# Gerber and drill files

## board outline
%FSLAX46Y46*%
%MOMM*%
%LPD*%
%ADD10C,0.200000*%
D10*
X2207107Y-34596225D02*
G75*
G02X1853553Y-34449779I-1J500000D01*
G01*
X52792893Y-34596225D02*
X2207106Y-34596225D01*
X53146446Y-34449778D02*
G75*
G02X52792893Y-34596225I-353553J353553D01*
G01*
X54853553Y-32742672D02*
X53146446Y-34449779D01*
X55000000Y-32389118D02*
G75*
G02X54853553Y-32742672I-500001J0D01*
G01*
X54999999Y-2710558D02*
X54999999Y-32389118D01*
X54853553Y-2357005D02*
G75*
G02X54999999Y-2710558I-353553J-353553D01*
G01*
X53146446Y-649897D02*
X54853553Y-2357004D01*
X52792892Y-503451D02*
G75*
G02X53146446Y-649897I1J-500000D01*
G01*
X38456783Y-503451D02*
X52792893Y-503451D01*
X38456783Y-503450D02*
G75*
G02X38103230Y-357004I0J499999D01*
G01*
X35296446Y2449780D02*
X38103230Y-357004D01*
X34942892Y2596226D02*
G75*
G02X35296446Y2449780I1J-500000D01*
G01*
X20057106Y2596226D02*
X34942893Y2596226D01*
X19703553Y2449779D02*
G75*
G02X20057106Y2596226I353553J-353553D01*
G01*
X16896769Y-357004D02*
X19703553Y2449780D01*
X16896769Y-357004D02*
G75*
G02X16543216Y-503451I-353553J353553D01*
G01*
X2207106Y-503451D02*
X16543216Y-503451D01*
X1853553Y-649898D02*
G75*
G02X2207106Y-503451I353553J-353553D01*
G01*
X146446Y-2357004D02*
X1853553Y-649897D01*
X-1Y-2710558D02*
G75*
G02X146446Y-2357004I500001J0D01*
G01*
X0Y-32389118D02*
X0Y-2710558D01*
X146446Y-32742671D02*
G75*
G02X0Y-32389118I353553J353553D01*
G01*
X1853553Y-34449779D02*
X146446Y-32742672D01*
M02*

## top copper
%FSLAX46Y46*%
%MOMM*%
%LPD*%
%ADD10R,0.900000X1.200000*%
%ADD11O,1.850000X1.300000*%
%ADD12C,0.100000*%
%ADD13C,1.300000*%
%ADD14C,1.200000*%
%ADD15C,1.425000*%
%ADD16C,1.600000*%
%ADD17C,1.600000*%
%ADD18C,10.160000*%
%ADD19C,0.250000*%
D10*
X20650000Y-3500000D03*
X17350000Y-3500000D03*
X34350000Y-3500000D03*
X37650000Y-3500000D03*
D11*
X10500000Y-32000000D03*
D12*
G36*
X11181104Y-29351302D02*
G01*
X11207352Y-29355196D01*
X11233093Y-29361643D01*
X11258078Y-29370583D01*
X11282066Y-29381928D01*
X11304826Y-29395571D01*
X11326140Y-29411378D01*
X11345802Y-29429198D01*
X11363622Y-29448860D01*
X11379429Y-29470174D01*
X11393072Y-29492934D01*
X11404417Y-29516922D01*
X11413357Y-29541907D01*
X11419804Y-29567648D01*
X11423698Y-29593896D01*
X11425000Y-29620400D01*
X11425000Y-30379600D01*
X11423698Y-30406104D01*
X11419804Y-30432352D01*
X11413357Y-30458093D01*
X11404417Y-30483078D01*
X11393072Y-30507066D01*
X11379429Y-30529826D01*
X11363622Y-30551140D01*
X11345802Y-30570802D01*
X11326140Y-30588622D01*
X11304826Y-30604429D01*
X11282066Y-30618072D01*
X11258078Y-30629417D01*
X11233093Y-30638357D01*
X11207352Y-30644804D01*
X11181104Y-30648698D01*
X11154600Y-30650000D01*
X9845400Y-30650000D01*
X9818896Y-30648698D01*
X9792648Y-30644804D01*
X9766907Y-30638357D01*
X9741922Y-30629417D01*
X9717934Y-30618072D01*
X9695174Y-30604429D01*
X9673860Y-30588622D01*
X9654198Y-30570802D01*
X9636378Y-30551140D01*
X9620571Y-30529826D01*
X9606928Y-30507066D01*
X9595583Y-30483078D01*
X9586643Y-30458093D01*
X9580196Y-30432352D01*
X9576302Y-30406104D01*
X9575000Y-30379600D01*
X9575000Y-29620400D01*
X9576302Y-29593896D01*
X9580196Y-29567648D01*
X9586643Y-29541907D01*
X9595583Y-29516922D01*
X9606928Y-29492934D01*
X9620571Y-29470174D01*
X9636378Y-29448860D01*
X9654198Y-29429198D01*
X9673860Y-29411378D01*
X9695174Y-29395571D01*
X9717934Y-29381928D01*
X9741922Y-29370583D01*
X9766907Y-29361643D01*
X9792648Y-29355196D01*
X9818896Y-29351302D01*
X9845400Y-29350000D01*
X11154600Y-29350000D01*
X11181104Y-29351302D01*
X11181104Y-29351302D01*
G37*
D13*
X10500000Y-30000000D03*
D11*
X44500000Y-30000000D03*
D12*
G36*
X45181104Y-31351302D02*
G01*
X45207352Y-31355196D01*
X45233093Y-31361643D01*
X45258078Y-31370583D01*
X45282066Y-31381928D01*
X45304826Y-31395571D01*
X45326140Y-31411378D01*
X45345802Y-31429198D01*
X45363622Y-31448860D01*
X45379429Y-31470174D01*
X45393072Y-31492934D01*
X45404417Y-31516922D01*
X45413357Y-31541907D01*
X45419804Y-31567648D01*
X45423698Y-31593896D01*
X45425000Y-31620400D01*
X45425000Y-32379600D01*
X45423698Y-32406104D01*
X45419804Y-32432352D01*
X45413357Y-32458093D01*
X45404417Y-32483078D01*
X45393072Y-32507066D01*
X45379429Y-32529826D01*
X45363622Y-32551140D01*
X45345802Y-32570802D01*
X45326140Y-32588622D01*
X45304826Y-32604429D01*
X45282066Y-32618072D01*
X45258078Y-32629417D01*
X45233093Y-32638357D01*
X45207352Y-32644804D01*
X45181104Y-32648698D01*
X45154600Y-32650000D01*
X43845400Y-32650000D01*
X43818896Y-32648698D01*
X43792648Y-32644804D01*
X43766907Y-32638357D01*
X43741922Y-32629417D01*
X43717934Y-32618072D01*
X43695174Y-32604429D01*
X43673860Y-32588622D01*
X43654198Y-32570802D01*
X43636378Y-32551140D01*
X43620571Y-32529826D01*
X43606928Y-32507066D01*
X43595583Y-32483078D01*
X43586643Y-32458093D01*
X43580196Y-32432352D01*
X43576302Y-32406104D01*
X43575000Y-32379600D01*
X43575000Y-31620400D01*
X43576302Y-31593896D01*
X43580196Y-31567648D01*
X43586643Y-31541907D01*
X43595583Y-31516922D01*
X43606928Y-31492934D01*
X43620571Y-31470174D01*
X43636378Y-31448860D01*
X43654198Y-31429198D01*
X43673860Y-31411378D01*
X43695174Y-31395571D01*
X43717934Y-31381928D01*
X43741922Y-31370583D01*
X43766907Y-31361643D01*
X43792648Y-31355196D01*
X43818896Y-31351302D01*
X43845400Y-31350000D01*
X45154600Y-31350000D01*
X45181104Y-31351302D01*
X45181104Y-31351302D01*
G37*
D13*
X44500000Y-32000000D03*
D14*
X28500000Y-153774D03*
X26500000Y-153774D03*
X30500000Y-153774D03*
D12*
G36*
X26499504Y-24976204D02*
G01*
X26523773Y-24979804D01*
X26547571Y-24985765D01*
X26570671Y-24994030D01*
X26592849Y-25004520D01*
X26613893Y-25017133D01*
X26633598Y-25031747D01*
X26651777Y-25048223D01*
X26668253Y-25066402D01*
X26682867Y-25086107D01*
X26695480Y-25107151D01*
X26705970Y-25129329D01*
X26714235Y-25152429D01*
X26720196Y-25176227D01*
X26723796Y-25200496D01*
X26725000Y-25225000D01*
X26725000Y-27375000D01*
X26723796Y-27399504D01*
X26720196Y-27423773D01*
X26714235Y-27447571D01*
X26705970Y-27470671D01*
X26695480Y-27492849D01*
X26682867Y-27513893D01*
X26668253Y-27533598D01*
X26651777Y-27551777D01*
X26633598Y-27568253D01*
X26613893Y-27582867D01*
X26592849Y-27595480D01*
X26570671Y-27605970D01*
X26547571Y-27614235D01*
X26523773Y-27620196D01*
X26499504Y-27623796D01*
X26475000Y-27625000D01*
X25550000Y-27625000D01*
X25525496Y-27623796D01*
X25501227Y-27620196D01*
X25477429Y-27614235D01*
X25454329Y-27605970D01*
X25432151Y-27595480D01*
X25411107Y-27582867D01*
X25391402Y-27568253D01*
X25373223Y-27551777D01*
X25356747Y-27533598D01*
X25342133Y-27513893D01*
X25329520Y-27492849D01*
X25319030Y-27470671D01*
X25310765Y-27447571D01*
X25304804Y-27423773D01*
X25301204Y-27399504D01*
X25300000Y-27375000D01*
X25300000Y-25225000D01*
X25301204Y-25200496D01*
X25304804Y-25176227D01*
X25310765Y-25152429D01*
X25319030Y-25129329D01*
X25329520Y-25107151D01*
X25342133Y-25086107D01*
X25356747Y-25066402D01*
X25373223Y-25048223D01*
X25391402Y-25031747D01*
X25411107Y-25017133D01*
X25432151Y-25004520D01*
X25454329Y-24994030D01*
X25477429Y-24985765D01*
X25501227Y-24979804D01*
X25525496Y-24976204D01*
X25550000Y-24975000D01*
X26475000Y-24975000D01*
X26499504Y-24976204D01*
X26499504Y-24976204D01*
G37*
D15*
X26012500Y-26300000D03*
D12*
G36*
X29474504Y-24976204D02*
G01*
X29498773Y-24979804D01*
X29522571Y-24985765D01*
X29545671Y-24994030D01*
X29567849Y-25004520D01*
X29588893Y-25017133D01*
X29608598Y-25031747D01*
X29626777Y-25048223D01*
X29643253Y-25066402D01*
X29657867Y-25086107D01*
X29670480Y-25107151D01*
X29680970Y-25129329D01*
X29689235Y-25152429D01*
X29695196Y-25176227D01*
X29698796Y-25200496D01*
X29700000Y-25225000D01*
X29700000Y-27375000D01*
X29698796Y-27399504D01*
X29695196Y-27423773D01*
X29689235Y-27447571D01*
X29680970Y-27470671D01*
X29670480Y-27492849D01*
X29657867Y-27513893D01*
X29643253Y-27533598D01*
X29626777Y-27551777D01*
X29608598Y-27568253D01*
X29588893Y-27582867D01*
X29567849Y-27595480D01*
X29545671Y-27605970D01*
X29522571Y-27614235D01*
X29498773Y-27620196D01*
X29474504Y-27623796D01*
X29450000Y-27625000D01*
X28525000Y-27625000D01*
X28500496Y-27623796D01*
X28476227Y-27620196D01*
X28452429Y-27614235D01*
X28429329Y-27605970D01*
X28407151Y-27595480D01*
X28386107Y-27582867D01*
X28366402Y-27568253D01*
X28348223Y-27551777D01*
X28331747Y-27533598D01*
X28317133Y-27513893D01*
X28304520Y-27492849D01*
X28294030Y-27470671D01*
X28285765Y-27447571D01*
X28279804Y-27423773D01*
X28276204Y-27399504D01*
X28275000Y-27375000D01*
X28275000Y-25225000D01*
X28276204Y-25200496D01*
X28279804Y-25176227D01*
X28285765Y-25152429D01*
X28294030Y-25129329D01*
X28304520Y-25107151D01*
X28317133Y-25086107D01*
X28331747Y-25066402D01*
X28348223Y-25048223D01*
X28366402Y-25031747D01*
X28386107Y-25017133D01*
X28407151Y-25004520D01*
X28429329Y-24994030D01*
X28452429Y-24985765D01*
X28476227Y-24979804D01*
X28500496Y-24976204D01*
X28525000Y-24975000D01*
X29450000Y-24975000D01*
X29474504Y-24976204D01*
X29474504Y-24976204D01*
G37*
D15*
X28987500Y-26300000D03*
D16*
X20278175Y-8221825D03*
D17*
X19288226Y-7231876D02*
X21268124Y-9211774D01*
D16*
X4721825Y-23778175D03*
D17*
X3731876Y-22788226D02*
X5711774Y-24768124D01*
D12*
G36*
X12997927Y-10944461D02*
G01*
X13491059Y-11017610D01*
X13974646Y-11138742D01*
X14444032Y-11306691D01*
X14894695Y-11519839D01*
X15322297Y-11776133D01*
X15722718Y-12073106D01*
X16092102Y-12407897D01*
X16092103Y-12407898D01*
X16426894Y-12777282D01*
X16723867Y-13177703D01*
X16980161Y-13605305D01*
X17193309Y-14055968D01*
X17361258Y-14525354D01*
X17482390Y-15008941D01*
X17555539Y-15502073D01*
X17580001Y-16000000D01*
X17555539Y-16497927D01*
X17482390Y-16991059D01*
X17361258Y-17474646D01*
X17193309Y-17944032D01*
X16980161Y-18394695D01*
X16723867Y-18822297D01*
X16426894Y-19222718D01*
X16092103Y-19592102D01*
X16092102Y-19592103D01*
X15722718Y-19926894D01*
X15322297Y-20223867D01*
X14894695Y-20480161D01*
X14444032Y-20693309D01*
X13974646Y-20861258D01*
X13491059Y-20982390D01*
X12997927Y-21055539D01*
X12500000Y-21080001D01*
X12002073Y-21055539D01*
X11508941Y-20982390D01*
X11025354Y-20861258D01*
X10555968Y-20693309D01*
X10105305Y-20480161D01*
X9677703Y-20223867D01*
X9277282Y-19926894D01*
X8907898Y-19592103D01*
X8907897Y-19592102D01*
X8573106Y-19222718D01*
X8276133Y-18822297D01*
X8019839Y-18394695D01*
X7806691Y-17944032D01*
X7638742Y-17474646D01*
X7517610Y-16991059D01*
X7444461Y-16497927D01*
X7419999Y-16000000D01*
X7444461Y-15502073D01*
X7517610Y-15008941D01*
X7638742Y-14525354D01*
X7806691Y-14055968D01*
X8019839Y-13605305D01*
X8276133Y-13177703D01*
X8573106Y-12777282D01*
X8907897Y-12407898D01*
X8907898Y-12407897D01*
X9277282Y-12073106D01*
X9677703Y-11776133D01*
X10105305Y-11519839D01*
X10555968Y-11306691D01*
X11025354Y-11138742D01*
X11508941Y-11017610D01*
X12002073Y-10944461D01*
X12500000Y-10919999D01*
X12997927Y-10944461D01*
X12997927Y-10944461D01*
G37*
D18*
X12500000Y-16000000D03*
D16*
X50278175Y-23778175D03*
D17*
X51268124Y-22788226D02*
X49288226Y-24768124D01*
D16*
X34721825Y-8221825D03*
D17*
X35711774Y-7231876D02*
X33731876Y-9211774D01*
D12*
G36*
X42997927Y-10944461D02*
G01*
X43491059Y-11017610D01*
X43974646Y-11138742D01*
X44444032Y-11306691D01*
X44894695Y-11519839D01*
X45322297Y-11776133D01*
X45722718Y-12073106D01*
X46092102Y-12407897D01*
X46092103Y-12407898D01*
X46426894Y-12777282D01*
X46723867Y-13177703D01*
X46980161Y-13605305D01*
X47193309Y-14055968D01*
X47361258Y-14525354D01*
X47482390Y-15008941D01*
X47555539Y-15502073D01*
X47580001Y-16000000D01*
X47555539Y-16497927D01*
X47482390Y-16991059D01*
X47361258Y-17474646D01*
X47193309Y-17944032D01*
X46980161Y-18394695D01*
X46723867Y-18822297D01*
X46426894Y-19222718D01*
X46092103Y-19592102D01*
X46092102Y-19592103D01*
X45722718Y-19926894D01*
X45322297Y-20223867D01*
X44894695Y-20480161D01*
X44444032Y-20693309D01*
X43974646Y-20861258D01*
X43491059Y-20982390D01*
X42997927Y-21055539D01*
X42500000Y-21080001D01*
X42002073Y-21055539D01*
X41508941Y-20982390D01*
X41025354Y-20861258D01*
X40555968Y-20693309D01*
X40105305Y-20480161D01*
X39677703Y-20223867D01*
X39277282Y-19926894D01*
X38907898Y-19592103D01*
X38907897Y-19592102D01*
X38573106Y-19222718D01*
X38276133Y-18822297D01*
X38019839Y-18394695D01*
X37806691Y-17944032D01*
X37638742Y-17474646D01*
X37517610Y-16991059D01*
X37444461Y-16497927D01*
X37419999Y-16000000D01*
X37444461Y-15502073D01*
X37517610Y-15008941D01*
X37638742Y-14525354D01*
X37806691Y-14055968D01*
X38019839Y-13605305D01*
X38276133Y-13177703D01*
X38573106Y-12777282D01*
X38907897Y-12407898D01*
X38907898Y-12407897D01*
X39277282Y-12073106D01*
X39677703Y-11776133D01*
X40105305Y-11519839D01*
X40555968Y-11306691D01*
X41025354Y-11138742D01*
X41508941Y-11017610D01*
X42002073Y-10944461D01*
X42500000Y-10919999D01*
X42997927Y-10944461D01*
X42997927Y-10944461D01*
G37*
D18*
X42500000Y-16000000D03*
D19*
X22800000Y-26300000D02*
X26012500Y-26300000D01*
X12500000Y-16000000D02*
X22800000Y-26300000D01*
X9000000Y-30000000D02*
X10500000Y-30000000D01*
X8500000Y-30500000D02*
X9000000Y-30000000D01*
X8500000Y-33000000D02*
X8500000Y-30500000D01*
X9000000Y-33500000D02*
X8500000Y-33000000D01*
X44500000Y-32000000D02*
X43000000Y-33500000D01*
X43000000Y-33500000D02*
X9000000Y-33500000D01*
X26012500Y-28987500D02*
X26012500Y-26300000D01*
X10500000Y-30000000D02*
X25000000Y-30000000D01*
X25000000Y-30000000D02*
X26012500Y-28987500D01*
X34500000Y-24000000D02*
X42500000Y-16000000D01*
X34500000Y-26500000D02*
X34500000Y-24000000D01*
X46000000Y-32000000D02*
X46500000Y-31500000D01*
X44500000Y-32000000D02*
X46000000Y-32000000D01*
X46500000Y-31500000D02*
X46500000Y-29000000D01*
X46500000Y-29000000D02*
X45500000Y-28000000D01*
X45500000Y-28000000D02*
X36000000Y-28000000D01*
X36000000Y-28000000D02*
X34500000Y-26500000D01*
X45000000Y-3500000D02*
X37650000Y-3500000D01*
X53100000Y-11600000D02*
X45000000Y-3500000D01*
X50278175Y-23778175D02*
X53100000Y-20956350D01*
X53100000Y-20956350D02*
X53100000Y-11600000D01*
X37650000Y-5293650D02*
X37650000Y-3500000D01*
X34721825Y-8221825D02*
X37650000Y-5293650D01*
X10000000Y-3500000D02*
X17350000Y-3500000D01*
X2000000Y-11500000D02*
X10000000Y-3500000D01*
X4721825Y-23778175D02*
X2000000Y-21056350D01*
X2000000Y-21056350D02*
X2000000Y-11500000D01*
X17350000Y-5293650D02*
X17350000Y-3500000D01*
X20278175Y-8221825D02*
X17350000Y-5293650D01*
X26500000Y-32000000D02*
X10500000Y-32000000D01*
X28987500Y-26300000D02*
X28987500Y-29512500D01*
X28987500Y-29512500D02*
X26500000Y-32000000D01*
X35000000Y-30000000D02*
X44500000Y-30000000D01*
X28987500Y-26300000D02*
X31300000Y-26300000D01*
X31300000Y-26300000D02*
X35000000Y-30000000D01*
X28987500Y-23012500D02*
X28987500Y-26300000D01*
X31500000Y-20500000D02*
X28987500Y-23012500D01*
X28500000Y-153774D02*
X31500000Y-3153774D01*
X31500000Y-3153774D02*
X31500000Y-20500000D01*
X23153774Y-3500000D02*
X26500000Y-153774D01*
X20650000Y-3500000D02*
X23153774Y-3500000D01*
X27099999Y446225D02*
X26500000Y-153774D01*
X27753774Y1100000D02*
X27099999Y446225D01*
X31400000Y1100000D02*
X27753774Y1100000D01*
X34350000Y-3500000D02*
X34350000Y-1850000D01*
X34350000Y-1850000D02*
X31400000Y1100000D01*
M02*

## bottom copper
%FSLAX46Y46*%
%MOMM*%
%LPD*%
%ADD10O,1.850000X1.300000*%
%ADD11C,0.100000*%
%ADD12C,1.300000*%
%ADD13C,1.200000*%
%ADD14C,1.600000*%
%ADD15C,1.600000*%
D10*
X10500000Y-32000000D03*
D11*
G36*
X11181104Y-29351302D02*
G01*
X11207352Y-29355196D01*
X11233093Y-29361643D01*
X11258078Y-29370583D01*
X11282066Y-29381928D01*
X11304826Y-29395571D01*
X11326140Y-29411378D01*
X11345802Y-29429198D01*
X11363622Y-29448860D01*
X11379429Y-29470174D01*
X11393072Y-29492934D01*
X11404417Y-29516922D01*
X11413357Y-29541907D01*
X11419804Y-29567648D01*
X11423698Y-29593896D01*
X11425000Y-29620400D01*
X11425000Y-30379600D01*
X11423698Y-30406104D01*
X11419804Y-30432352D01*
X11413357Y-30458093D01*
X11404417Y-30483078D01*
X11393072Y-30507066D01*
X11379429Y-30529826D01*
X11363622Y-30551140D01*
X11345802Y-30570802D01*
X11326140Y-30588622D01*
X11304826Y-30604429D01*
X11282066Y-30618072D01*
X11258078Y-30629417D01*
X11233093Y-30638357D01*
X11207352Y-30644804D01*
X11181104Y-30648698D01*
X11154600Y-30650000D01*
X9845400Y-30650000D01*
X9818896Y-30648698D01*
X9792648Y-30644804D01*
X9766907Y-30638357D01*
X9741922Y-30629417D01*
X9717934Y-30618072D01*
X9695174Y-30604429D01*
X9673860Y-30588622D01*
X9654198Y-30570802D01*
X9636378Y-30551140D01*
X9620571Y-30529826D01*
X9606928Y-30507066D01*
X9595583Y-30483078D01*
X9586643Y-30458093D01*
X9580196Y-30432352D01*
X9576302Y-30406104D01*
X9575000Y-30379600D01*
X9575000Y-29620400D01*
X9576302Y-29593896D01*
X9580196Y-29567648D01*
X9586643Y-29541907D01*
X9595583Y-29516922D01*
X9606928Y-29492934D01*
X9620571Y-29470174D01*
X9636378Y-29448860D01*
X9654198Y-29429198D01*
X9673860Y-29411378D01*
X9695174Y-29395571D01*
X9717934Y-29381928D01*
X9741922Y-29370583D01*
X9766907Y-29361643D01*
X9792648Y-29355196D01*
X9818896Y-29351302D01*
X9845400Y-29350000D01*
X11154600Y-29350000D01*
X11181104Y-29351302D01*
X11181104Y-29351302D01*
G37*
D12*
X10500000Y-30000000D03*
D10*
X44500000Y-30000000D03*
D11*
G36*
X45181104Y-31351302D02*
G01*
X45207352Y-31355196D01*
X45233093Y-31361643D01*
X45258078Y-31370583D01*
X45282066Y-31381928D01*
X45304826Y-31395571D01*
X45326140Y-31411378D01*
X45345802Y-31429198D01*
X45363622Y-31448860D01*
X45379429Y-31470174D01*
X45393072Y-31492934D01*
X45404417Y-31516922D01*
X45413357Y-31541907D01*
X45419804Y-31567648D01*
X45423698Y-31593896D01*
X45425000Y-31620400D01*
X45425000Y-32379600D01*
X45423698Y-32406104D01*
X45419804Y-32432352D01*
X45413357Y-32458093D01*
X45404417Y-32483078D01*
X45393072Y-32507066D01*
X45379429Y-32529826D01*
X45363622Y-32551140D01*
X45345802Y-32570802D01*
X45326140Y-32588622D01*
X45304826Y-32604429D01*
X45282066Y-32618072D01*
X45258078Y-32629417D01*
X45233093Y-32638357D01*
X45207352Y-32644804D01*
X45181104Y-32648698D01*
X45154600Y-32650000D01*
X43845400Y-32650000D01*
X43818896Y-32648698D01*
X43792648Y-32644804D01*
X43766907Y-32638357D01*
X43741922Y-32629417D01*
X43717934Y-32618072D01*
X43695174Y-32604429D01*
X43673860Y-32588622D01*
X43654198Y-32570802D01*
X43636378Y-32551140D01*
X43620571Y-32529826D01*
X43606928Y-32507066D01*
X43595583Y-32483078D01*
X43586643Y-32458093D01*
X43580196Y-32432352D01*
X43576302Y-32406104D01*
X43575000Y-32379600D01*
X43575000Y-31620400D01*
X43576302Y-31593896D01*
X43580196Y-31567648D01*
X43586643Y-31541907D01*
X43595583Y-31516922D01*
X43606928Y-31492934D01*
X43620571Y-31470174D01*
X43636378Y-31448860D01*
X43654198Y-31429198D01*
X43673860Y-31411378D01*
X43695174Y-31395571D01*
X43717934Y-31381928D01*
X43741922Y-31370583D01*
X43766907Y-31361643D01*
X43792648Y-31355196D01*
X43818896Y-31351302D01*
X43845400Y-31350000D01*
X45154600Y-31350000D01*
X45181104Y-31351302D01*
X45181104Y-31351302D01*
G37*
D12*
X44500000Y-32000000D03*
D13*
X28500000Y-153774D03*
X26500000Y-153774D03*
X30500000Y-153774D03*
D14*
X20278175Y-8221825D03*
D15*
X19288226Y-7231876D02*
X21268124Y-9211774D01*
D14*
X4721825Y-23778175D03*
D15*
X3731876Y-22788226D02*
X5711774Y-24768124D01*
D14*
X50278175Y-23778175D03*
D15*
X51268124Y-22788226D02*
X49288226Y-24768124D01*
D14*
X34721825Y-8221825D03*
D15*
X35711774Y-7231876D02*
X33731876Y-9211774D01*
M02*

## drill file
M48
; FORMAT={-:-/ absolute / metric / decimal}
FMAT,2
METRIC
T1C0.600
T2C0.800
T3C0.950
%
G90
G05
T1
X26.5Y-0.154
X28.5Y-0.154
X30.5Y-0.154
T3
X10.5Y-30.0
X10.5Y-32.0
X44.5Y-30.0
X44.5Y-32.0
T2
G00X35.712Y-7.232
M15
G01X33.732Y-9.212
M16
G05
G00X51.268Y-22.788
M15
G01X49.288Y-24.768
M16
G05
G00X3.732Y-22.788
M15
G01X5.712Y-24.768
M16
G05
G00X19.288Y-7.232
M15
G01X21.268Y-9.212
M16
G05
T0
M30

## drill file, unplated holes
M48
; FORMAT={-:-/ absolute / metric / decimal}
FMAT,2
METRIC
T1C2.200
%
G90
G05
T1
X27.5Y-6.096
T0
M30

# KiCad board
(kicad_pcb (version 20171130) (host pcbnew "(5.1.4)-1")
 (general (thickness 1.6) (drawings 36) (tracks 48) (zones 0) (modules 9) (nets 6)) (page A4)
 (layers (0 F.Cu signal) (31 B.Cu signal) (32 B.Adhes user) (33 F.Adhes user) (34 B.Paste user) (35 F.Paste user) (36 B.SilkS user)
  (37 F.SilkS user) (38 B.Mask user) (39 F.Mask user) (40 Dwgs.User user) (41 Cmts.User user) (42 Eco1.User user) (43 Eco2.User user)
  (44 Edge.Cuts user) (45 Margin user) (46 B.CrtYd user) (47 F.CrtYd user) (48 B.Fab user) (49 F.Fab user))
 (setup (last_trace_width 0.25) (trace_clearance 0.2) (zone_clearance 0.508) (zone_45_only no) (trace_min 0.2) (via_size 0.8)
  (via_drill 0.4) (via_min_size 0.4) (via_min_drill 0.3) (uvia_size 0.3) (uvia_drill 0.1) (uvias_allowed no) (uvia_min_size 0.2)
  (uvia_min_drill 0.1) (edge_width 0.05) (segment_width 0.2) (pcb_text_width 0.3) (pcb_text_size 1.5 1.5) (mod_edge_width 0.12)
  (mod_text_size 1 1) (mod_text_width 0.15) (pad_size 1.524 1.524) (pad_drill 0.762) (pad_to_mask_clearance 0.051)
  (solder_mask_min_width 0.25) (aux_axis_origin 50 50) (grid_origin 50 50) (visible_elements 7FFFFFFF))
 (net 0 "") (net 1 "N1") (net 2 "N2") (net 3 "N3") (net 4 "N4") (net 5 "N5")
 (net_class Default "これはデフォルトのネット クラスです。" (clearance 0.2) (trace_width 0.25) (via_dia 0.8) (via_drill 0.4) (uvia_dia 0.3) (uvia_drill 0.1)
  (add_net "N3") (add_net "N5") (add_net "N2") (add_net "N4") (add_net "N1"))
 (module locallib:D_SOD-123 (layer F.Cu) (at 69 53.5 180)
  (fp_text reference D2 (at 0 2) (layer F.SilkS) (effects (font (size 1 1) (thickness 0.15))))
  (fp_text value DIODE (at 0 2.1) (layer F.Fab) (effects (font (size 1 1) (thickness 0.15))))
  (pad 1 smd rect (at -1.65 0 180) (size 0.9 1.2) (layers F.Cu F.Paste F.Mask) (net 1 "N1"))
  (pad 2 smd rect (at 1.65 0 180) (size 0.9 1.2) (layers F.Cu F.Paste F.Mask) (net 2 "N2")))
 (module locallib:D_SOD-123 (layer F.Cu) (at 86 53.5)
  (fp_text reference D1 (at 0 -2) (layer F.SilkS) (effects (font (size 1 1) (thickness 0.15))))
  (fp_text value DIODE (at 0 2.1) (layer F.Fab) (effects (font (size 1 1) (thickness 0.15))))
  (pad 1 smd rect (at -1.65 0) (size 0.9 1.2) (layers F.Cu F.Paste F.Mask) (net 1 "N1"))
  (pad 2 smd rect (at 1.65 0) (size 0.9 1.2) (layers F.Cu F.Paste F.Mask) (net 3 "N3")))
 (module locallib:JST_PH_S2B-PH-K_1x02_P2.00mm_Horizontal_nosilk (layer F.Cu) (at 60.5 80 270)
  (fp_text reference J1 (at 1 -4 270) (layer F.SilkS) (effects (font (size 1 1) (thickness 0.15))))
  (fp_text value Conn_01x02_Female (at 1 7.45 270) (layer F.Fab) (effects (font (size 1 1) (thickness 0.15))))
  (pad 2 thru_hole oval (at 2 0 270) (size 1.3 1.85) (drill 0.95) (layers *.Cu *.Mask) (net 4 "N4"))
  (pad 1 thru_hole roundrect (at 0 0 270) (size 1.3 1.85) (drill 0.95) (layers *.Cu *.Mask) (roundrect_rratio 0.208) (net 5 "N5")))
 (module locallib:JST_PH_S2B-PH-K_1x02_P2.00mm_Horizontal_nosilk (layer F.Cu) (at 94.5 82 90)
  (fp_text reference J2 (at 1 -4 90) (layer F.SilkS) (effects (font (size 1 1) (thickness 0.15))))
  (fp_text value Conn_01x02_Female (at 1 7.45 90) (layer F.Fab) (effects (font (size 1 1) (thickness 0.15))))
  (pad 2 thru_hole oval (at 2 0 90) (size 1.3 1.85) (drill 0.95) (layers *.Cu *.Mask) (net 4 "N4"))
  (pad 1 thru_hole roundrect (at 0 0 90) (size 1.3 1.85) (drill 0.95) (layers *.Cu *.Mask) (roundrect_rratio 0.208) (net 5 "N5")))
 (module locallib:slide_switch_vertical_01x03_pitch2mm (layer B.Cu) (at 80.5 50.153774 90)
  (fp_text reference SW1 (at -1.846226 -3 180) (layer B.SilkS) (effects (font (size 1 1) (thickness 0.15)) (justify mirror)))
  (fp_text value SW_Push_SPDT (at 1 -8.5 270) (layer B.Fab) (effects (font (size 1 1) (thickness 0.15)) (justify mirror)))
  (pad 3 thru_hole circle (at 0 -2 90) (size 1.2 1.2) (drill 0.6) (layers *.Cu *.Mask) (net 4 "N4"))
  (pad 2 thru_hole circle (at 0 -4 90) (size 1.2 1.2) (drill 0.6) (layers *.Cu *.Mask) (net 1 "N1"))
  (pad 1 thru_hole circle (at 0 0 90) (size 1.2 1.2) (drill 0.6) (layers *.Cu *.Mask)))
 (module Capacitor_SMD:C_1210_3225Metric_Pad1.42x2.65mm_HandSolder (layer F.Cu) (at 77.5 76.3 180)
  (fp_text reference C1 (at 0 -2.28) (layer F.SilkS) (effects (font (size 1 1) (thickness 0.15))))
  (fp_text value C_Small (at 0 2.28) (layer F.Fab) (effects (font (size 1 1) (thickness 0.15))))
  (pad 2 smd roundrect (at 1.4875 0 180) (size 1.425 2.65) (layers F.Cu F.Paste F.Mask) (roundrect_rratio 0.175439) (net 5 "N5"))
  (pad 1 smd roundrect (at -1.4875 0 180) (size 1.425 2.65) (layers F.Cu F.Paste F.Mask) (roundrect_rratio 0.175439) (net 4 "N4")))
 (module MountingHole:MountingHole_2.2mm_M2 (layer F.Cu) (at 77.5 56.096225)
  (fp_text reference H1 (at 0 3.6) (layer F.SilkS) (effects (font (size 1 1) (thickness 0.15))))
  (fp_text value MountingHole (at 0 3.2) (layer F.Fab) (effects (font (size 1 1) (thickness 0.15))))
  (pad 1 np_thru_hole circle (at 0 0) (size 2.2 2.2) (drill 2.2) (layers *.Cu *.Mask)))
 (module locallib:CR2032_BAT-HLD (layer F.Cu) (at 62.5 66 45)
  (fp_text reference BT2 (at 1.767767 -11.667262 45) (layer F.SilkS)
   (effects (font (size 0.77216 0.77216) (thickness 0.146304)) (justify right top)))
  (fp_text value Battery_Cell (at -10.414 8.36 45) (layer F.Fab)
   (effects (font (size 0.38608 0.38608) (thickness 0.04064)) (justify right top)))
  (pad 1 thru_hole oval (at 11 0 45) (size 1.6 4.4) (drill oval 0.8 3.6) (layers *.Cu *.Mask) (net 2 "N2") (solder_mask_margin 0.1016))
  (pad 1 thru_hole oval (at -11 0 45) (size 1.6 4.4) (drill oval 0.8 3.6) (layers *.Cu *.Mask) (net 2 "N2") (solder_mask_margin 0.1016))
  (pad 2 smd roundrect (at 0 0 45) (size 10.16 10.16) (layers F.Cu F.Mask) (roundrect_rratio 0.5) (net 5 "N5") (solder_mask_margin 0.1016)))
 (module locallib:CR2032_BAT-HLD (layer F.Cu) (at 92.5 66 315)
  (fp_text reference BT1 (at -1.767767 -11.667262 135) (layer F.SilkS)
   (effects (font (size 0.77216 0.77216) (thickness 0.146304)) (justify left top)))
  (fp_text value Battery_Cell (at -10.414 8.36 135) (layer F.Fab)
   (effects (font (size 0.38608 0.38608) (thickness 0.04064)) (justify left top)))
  (pad 1 thru_hole oval (at 11 0 315) (size 1.6 4.4) (drill oval 0.8 3.6) (layers *.Cu *.Mask) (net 3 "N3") (solder_mask_margin 0.1016))
  (pad 1 thru_hole oval (at -11 0 315) (size 1.6 4.4) (drill oval 0.8 3.6) (layers *.Cu *.Mask) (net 3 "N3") (solder_mask_margin 0.1016))
  (pad 2 smd roundrect (at 0 0 315) (size 10.16 10.16) (layers F.Cu F.Mask) (roundrect_rratio 0.5) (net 5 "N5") (solder_mask_margin 0.1016)))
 (gr_arc (start 52.207106 84.096225) (end 51.853553 84.449779) (angle -45) (layer Edge.Cuts) (width 0.2))
 (gr_line (start 102.792893 84.596225) (end 52.207106 84.596225) (layer Edge.Cuts) (width 0.2))
 (gr_arc (start 102.792893 84.096225) (end 102.792893 84.596225) (angle -45) (layer Edge.Cuts) (width 0.2))
 (gr_line (start 104.853553 82.742672) (end 103.146446 84.449779) (layer Edge.Cuts) (width 0.2))
 (gr_arc (start 104.499999 82.389118) (end 104.853553 82.742672) (angle -45) (layer Edge.Cuts) (width 0.2))
 (gr_line (start 104.999999 52.710558) (end 104.999999 82.389118) (layer Edge.Cuts) (width 0.2))
 (gr_arc (start 104.5 52.710558) (end 104.999999 52.710558) (angle -45) (layer Edge.Cuts) (width 0.2))
 (gr_line (start 103.146446 50.649897) (end 104.853553 52.357004) (layer Edge.Cuts) (width 0.2))
 (gr_arc (start 102.792893 51.003451) (end 103.146446 50.649897) (angle -45) (layer Edge.Cuts) (width 0.2))
 (gr_line (start 88.456783 50.503451) (end 102.792893 50.503451) (layer Edge.Cuts) (width 0.2))
 (gr_arc (start 88.456783 50.003451) (end 88.10323 50.357004) (angle -45) (layer Edge.Cuts) (width 0.2))
 (gr_line (start 85.296446 47.55022) (end 88.10323 50.357004) (layer Edge.Cuts) (width 0.2))
 (gr_arc (start 84.942893 47.903774) (end 85.296446 47.55022) (angle -45) (layer Edge.Cuts) (width 0.2))
 (gr_line (start 70.057106 47.403774) (end 84.942893 47.403774) (layer Edge.Cuts) (width 0.2))
 (gr_arc (start 70.057106 47.903774) (end 70.057106 47.403774) (angle -45) (layer Edge.Cuts) (width 0.2))
 (gr_line (start 66.896769 50.357004) (end 69.703553 47.55022) (layer Edge.Cuts) (width 0.2))
 (gr_arc (start 66.543216 50.003451) (end 66.543216 50.503451) (angle -45) (layer Edge.Cuts) (width 0.2))
 (gr_line (start 52.207106 50.503451) (end 66.543216 50.503451) (layer Edge.Cuts) (width 0.2))
 (gr_arc (start 52.207106 51.003451) (end 52.207106 50.503451) (angle -45) (layer Edge.Cuts) (width 0.2))
 (gr_line (start 50.146446 52.357004) (end 51.853553 50.649897) (layer Edge.Cuts) (width 0.2))
 (gr_arc (start 50.5 52.710558) (end 50.146446 52.357004) (angle -45) (layer Edge.Cuts) (width 0.2))
 (gr_line (start 50 82.389118) (end 50 52.710558) (layer Edge.Cuts) (width 0.2))
 (gr_arc (start 50.499999 82.389118) (end 50 82.389118) (angle -45) (layer Edge.Cuts) (width 0.2))
 (gr_line (start 51.853553 84.449779) (end 50.146446 82.742672) (layer Edge.Cuts) (width 0.2))
 (segment (start 72.8 76.3) (end 76.0125 76.3) (width 0.25) (layer F.Cu) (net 5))
 (segment (start 62.5 66) (end 72.8 76.3) (width 0.25) (layer F.Cu) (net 5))
 (segment (start 59 80) (end 60.5 80) (width 0.25) (layer F.Cu) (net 5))
 (segment (start 58.5 80.5) (end 59 80) (width 0.25) (layer F.Cu) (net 5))
 (segment (start 58.5 83) (end 58.5 80.5) (width 0.25) (layer F.Cu) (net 5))
 (segment (start 59 83.5) (end 58.5 83) (width 0.25) (layer F.Cu) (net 5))
 (segment (start 94.5 82) (end 93 83.5) (width 0.25) (layer F.Cu) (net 5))
 (segment (start 93 83.5) (end 59 83.5) (width 0.25) (layer F.Cu) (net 5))
 (segment (start 76.0125 78.9875) (end 76.0125 76.3) (width 0.25) (layer F.Cu) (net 5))
 (segment (start 60.5 80) (end 75 80) (width 0.25) (layer F.Cu) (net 5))
 (segment (start 75 80) (end 76.0125 78.9875) (width 0.25) (layer F.Cu) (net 5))
 (segment (start 84.5 74) (end 92.5 66) (width 0.25) (layer F.Cu) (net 5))
 (segment (start 84.5 76.5) (end 84.5 74) (width 0.25) (layer F.Cu) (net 5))
 (segment (start 96 82) (end 96.5 81.5) (width 0.25) (layer F.Cu) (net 5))
 (segment (start 94.5 82) (end 96 82) (width 0.25) (layer F.Cu) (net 5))
 (segment (start 96.5 81.5) (end 96.5 79) (width 0.25) (layer F.Cu) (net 5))
 (segment (start 96.5 79) (end 95.5 78) (width 0.25) (layer F.Cu) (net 5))
 (segment (start 95.5 78) (end 86 78) (width 0.25) (layer F.Cu) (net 5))
 (segment (start 86 78) (end 84.5 76.5) (width 0.25) (layer F.Cu) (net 5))
 (segment (start 95 53.5) (end 87.65 53.5) (width 0.25) (layer F.Cu) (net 3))
 (segment (start 103.1 61.6) (end 95 53.5) (width 0.25) (layer F.Cu) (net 3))
 (segment (start 100.278175 73.778175) (end 103.1 70.95635) (width 0.25) (layer F.Cu) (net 3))
 (segment (start 103.1 70.95635) (end 103.1 61.6) (width 0.25) (layer F.Cu) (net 3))
 (segment (start 87.65 55.29365) (end 87.65 53.5) (width 0.25) (layer F.Cu) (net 3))
 (segment (start 84.721825 58.221825) (end 87.65 55.29365) (width 0.25) (layer F.Cu) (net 3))
 (segment (start 60 53.5) (end 67.35 53.5) (width 0.25) (layer F.Cu) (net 2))
 (segment (start 52 61.5) (end 60 53.5) (width 0.25) (layer F.Cu) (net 2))
 (segment (start 54.721825 73.778175) (end 52 71.05635) (width 0.25) (layer F.Cu) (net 2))
 (segment (start 52 71.05635) (end 52 61.5) (width 0.25) (layer F.Cu) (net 2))
 (segment (start 67.35 55.29365) (end 67.35 53.5) (width 0.25) (layer F.Cu) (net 2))
 (segment (start 70.278175 58.221825) (end 67.35 55.29365) (width 0.25) (layer F.Cu) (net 2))
 (segment (start 76.5 82) (end 60.5 82) (width 0.25) (layer F.Cu) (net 4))
 (segment (start 78.9875 76.3) (end 78.9875 79.5125) (width 0.25) (layer F.Cu) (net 4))
 (segment (start 78.9875 79.5125) (end 76.5 82) (width 0.25) (layer F.Cu) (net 4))
 (segment (start 85 80) (end 94.5 80) (width 0.25) (layer F.Cu) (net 4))
 (segment (start 78.9875 76.3) (end 81.3 76.3) (width 0.25) (layer F.Cu) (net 4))
 (segment (start 81.3 76.3) (end 85 80) (width 0.25) (layer F.Cu) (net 4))
 (segment (start 78.9875 73.0125) (end 78.9875 76.3) (width 0.25) (layer F.Cu) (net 4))
 (segment (start 81.5 70.5) (end 78.9875 73.0125) (width 0.25) (layer F.Cu) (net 4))
 (segment (start 78.5 50.153774) (end 81.5 53.153774) (width 0.25) (layer F.Cu) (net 4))
 (segment (start 81.5 53.153774) (end 81.5 70.5) (width 0.25) (layer F.Cu) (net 4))
 (segment (start 73.153774 53.5) (end 76.5 50.153774) (width 0.25) (layer F.Cu) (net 1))
 (segment (start 70.65 53.5) (end 73.153774 53.5) (width 0.25) (layer F.Cu) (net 1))
 (segment (start 77.099999 49.553775) (end 76.5 50.153774) (width 0.25) (layer F.Cu) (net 1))
 (segment (start 77.753774 48.9) (end 77.099999 49.553775) (width 0.25) (layer F.Cu) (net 1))
 (segment (start 81.4 48.9) (end 77.753774 48.9) (width 0.25) (layer F.Cu) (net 1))
 (segment (start 84.35 53.5) (end 84.35 51.85) (width 0.25) (layer F.Cu) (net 1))
 (segment (start 84.35 51.85) (end 81.4 48.9) (width 0.25) (layer F.Cu) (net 1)))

